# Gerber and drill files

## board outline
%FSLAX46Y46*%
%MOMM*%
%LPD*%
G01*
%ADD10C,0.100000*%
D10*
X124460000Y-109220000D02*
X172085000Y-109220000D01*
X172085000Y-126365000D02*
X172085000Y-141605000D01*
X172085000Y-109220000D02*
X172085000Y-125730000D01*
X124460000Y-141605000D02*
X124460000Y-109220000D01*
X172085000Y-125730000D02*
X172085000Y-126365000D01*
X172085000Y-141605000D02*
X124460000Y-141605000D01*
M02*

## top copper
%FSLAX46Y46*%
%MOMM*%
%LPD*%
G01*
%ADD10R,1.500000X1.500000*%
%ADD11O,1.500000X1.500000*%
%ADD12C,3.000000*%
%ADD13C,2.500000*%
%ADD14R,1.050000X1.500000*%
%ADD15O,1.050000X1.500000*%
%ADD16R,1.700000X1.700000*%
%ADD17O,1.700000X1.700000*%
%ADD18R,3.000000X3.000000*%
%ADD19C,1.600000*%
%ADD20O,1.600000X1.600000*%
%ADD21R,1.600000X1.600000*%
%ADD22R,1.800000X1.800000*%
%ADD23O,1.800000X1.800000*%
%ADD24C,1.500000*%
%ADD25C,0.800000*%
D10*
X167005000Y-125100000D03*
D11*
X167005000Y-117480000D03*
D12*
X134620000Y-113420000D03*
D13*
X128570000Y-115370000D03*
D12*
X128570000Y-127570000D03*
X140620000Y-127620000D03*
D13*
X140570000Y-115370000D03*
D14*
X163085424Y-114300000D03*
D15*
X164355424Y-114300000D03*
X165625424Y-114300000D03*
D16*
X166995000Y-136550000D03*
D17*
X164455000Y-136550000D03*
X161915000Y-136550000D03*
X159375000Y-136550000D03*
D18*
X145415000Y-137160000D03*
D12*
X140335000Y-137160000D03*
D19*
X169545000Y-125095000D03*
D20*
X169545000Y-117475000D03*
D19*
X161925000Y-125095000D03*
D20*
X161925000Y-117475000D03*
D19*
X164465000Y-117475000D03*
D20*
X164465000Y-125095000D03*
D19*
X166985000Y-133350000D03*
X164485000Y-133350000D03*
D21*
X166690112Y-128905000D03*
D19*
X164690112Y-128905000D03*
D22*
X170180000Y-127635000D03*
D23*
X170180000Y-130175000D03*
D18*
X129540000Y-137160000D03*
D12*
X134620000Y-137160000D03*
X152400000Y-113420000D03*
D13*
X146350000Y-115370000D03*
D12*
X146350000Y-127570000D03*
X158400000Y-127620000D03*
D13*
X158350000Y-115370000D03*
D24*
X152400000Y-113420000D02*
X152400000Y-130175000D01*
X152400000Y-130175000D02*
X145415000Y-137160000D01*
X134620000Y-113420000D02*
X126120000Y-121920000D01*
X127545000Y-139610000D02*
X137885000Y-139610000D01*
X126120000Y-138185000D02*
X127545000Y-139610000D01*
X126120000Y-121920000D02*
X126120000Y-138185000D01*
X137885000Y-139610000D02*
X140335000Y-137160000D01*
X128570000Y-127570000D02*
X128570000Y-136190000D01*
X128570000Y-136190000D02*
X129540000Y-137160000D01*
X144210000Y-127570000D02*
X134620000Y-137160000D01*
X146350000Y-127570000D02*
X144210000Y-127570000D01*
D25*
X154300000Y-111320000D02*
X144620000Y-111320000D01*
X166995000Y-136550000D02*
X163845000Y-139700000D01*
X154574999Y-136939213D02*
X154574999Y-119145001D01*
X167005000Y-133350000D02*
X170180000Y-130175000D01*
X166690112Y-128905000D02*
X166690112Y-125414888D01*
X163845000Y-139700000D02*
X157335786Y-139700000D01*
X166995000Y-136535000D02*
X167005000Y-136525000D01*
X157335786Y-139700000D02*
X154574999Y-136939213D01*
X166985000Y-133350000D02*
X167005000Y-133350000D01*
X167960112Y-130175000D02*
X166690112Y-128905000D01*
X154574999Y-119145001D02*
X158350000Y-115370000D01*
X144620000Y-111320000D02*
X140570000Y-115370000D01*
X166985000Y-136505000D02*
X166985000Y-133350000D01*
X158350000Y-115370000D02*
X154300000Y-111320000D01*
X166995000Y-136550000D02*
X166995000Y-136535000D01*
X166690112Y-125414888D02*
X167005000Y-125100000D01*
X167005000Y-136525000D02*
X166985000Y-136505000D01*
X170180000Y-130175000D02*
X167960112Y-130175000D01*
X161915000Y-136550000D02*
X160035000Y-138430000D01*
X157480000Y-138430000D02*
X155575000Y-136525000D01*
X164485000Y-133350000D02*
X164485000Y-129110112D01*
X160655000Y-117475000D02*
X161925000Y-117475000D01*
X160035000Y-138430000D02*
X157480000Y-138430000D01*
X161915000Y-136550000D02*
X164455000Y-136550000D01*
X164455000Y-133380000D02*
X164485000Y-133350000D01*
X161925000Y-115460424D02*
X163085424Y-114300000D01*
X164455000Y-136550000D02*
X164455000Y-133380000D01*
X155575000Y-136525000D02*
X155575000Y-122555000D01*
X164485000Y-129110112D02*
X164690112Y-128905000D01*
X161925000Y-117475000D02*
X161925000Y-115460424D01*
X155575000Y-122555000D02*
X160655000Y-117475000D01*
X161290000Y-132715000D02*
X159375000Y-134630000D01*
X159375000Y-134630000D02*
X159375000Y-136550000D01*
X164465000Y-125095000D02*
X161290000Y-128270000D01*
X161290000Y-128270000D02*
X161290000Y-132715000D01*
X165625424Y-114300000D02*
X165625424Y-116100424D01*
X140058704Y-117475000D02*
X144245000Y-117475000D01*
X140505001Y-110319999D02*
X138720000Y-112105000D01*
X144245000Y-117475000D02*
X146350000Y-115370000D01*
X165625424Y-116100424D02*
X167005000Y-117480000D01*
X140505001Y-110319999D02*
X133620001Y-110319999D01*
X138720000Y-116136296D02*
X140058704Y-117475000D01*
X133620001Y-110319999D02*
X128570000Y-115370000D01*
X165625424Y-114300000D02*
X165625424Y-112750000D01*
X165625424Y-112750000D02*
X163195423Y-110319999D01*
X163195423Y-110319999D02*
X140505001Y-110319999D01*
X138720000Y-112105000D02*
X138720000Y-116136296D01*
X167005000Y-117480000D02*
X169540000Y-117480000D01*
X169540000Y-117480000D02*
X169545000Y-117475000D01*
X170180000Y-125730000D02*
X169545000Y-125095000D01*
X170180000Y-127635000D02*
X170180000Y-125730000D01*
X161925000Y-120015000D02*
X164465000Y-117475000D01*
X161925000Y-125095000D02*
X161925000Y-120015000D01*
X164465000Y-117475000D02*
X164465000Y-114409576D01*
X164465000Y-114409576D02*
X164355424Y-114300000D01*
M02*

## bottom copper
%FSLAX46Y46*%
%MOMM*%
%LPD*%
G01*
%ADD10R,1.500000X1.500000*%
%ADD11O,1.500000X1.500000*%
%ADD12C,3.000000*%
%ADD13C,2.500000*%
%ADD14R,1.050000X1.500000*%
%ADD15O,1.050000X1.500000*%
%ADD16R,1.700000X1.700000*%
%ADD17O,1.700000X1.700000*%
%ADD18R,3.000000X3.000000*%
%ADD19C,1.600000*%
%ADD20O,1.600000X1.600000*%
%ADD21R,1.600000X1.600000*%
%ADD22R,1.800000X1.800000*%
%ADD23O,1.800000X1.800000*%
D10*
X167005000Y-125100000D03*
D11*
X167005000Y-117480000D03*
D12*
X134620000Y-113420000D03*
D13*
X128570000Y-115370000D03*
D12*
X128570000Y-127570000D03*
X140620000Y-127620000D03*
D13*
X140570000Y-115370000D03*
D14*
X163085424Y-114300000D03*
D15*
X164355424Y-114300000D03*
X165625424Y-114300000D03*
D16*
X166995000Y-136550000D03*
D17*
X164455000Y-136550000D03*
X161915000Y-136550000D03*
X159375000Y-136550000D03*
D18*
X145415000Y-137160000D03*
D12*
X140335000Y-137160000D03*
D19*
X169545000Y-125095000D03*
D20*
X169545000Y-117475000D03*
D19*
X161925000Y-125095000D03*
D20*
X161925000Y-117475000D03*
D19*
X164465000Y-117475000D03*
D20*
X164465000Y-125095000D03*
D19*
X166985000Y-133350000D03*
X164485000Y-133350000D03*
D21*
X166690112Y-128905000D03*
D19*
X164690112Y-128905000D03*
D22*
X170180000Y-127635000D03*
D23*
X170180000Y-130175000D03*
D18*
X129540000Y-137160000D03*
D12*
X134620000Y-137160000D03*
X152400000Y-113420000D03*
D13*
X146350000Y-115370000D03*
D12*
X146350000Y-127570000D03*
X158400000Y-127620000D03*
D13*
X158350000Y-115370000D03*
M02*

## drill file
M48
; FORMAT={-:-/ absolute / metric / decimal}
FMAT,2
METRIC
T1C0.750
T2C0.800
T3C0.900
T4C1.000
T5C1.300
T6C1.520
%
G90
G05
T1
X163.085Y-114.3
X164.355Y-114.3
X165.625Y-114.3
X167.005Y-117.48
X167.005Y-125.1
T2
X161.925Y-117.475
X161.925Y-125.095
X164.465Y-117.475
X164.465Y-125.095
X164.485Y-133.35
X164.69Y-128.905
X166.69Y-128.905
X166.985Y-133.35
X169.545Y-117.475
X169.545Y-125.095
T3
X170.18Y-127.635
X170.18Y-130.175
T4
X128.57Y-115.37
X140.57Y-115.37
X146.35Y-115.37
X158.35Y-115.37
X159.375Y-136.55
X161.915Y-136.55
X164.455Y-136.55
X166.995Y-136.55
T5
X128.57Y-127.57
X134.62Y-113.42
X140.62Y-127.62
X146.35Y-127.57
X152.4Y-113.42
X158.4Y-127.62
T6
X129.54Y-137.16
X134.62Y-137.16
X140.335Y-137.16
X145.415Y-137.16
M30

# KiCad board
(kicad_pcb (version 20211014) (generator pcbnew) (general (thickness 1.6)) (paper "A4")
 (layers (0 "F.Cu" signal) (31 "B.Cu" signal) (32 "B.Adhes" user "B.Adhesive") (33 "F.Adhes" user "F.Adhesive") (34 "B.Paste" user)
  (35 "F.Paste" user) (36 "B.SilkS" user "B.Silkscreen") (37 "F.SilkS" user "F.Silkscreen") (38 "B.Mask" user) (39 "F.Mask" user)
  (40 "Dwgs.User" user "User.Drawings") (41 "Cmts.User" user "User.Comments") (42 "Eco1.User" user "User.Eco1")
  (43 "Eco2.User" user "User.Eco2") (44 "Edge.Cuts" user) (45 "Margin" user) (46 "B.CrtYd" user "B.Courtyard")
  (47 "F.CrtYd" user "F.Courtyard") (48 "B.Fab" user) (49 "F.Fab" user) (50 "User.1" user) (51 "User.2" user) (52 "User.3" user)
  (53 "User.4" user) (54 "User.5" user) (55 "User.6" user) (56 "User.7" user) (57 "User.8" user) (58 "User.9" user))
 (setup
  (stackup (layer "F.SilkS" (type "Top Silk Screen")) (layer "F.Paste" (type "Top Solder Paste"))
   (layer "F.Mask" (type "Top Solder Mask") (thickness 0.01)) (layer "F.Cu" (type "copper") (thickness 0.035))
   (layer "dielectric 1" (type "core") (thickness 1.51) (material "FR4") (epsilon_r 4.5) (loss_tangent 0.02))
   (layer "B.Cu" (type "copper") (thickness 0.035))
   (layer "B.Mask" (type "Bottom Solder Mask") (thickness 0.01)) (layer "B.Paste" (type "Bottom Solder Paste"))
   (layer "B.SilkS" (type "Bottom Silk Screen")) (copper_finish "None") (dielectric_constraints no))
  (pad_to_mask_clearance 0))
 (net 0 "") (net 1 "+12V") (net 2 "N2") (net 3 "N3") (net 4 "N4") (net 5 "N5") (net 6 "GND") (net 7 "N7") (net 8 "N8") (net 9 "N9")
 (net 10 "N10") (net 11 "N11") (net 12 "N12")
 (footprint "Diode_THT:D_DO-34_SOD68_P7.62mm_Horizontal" (layer "F.Cu") (at 167.005 125.1 90)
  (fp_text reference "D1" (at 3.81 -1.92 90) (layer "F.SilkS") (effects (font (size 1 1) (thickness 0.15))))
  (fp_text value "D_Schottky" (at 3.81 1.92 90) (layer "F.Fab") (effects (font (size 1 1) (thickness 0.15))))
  (pad "1" thru_hole rect (at 0 0 90) (size 1.5 1.5) (drill 0.75) (layers *.Cu *.Mask) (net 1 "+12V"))
  (pad "2" thru_hole oval (at 7.62 0 90) (size 1.5 1.5) (drill 0.75) (layers *.Cu *.Mask) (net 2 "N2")))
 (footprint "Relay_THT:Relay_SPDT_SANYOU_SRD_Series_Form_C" (layer "F.Cu") (at 134.62 113.42 -90)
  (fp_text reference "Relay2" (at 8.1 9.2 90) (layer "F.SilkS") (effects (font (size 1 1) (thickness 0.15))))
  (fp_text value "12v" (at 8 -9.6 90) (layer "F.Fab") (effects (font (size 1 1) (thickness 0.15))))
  (pad "1" thru_hole circle (at 0 0) (size 3 3) (drill 1.3) (layers *.Cu *.Mask) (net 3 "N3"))
  (pad "2" thru_hole circle (at 1.95 6.05) (size 2.5 2.5) (drill 1) (layers *.Cu *.Mask) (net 2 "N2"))
  (pad "3" thru_hole circle (at 14.15 6.05) (size 3 3) (drill 1.3) (layers *.Cu *.Mask) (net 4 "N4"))
  (pad "4" thru_hole circle (at 14.2 -6) (size 3 3) (drill 1.3) (layers *.Cu *.Mask) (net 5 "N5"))
  (pad "5" thru_hole circle (at 1.95 -5.95) (size 2.5 2.5) (drill 1) (layers *.Cu *.Mask) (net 1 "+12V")))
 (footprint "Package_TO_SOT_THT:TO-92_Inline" (layer "F.Cu") (at 163.085424 114.3)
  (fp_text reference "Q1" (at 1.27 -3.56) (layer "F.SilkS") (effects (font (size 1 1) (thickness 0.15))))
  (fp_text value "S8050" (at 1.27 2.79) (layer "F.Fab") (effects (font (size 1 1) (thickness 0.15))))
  (pad "1" thru_hole rect (at 0 0) (size 1.05 1.5) (drill 0.75) (layers *.Cu *.Mask) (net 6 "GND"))
  (pad "2" thru_hole oval (at 1.27 0) (size 1.05 1.5) (drill 0.75) (layers *.Cu *.Mask) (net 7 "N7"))
  (pad "3" thru_hole oval (at 2.54 0) (size 1.05 1.5) (drill 0.75) (layers *.Cu *.Mask) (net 2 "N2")))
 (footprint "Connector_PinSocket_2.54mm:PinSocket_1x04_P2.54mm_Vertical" (layer "F.Cu") (at 166.995 136.55 -90)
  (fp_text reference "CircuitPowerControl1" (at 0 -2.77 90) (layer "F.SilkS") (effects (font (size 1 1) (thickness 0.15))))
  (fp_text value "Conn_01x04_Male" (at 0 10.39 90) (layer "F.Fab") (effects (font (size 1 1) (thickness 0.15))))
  (pad "1" thru_hole rect (at 0 0 270) (size 1.7 1.7) (drill 1) (layers *.Cu *.Mask) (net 1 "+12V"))
  (pad "2" thru_hole oval (at 0 2.54 270) (size 1.7 1.7) (drill 1) (layers *.Cu *.Mask) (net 6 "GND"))
  (pad "3" thru_hole oval (at 0 5.08 270) (size 1.7 1.7) (drill 1) (layers *.Cu *.Mask) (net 6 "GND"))
  (pad "4" thru_hole oval (at 0 7.62 270) (size 1.7 1.7) (drill 1) (layers *.Cu *.Mask) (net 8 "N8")))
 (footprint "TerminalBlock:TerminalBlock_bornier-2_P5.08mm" (layer "F.Cu") (at 145.415 137.16 180)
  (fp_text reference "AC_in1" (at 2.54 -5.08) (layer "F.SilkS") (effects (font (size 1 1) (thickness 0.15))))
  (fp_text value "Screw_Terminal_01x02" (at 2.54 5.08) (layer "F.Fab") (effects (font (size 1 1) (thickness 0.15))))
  (pad "1" thru_hole rect (at 0 0 180) (size 3 3) (drill 1.52) (layers *.Cu *.Mask) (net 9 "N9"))
  (pad "2" thru_hole circle (at 5.08 0 180) (size 3 3) (drill 1.52) (layers *.Cu *.Mask) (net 3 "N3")))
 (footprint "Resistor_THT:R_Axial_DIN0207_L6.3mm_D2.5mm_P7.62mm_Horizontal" (layer "F.Cu") (at 169.545 125.095 90)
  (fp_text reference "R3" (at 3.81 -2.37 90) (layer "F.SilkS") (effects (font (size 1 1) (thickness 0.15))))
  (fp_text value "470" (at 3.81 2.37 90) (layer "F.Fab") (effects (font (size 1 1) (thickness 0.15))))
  (pad "1" thru_hole circle (at 0 0 90) (size 1.6 1.6) (drill 0.8) (layers *.Cu *.Mask) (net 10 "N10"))
  (pad "2" thru_hole oval (at 7.62 0 90) (size 1.6 1.6) (drill 0.8) (layers *.Cu *.Mask) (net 2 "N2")))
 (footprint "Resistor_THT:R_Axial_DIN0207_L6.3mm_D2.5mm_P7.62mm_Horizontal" (layer "F.Cu") (at 161.925 125.095 90)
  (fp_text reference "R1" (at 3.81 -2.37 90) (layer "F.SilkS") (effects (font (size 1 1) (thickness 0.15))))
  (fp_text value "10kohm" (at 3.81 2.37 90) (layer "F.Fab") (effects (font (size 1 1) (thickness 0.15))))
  (pad "1" thru_hole circle (at 0 0 90) (size 1.6 1.6) (drill 0.8) (layers *.Cu *.Mask) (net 7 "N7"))
  (pad "2" thru_hole oval (at 7.62 0 90) (size 1.6 1.6) (drill 0.8) (layers *.Cu *.Mask) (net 6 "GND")))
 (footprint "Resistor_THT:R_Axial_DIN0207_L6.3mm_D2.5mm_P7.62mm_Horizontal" (layer "F.Cu") (at 164.465 117.475 -90)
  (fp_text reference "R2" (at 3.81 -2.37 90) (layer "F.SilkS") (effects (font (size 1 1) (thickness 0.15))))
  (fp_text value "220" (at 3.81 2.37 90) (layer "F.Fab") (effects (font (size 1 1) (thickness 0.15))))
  (pad "1" thru_hole circle (at 0 0 270) (size 1.6 1.6) (drill 0.8) (layers *.Cu *.Mask) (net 7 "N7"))
  (pad "2" thru_hole oval (at 7.62 0 270) (size 1.6 1.6) (drill 0.8) (layers *.Cu *.Mask) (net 8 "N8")))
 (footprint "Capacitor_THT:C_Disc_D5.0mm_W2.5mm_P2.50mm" (layer "F.Cu") (at 166.985 133.35 180)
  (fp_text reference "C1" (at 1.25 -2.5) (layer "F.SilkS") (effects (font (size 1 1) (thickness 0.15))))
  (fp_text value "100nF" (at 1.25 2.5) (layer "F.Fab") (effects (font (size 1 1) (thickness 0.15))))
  (pad "1" thru_hole circle (at 0 0 180) (size 1.6 1.6) (drill 0.8) (layers *.Cu *.Mask) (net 1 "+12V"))
  (pad "2" thru_hole circle (at 2.5 0 180) (size 1.6 1.6) (drill 0.8) (layers *.Cu *.Mask) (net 6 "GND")))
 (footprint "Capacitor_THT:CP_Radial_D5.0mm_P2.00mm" (layer "F.Cu") (at 166.690112 128.905 180)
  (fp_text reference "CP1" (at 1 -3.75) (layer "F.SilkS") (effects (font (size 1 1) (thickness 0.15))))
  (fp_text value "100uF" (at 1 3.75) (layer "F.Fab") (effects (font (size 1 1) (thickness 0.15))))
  (pad "1" thru_hole rect (at 0 0 180) (size 1.6 1.6) (drill 0.8) (layers *.Cu *.Mask) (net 1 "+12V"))
  (pad "2" thru_hole circle (at 2 0 180) (size 1.6 1.6) (drill 0.8) (layers *.Cu *.Mask) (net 6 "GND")))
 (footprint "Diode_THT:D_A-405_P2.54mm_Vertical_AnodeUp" (layer "F.Cu") (at 170.18 127.635 -90)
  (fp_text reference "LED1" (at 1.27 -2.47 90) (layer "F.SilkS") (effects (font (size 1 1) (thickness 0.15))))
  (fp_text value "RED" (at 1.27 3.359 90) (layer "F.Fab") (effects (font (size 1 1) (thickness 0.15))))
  (pad "1" thru_hole rect (at 0 0 270) (size 1.8 1.8) (drill 0.9) (layers *.Cu *.Mask) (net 10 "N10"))
  (pad "2" thru_hole oval (at 2.54 0 270) (size 1.8 1.8) (drill 0.9) (layers *.Cu *.Mask) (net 1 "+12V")))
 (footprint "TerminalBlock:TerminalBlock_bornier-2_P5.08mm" (layer "F.Cu") (at 129.54 137.16)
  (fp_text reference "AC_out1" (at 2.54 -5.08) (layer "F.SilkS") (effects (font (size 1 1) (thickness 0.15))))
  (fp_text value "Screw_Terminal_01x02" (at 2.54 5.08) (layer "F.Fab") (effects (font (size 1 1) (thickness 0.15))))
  (pad "1" thru_hole rect (at 0 0) (size 3 3) (drill 1.52) (layers *.Cu *.Mask) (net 4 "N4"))
  (pad "2" thru_hole circle (at 5.08 0) (size 3 3) (drill 1.52) (layers *.Cu *.Mask) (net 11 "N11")))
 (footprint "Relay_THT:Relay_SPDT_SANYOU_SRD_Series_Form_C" (layer "F.Cu") (at 152.4 113.42 -90)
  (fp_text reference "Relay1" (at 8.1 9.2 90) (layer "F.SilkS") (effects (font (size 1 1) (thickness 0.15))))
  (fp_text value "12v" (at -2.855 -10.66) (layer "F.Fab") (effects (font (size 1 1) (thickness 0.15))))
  (pad "1" thru_hole circle (at 0 0) (size 3 3) (drill 1.3) (layers *.Cu *.Mask) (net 9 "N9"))
  (pad "2" thru_hole circle (at 1.95 6.05) (size 2.5 2.5) (drill 1) (layers *.Cu *.Mask) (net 2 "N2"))
  (pad "3" thru_hole circle (at 14.15 6.05) (size 3 3) (drill 1.3) (layers *.Cu *.Mask) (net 11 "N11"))
  (pad "4" thru_hole circle (at 14.2 -6) (size 3 3) (drill 1.3) (layers *.Cu *.Mask) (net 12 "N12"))
  (pad "5" thru_hole circle (at 1.95 -5.95) (size 2.5 2.5) (drill 1) (layers *.Cu *.Mask) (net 1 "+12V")))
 (gr_line (start 124.46 109.22) (end 172.085 109.22) (layer "Edge.Cuts") (width 0.1))
 (gr_line (start 172.085 126.365) (end 172.085 141.605) (layer "Edge.Cuts") (width 0.1))
 (gr_line (start 172.085 109.22) (end 172.085 125.73) (layer "Edge.Cuts") (width 0.1))
 (gr_line (start 124.46 141.605) (end 124.46 109.22) (layer "Edge.Cuts") (width 0.1))
 (gr_line (start 172.085 125.73) (end 172.085 126.365) (layer "Edge.Cuts") (width 0.1))
 (gr_line (start 172.085 141.605) (end 124.46 141.605) (layer "Edge.Cuts") (width 0.1))
 (segment (start 152.4 113.42) (end 152.4 130.175) (width 1.5) (layer "F.Cu") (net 9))
 (segment (start 152.4 130.175) (end 145.415 137.16) (width 1.5) (layer "F.Cu") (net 9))
 (segment (start 134.62 113.42) (end 126.12 121.92) (width 1.5) (layer "F.Cu") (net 3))
 (segment (start 127.545 139.61) (end 137.885 139.61) (width 1.5) (layer "F.Cu") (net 3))
 (segment (start 126.12 138.185) (end 127.545 139.61) (width 1.5) (layer "F.Cu") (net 3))
 (segment (start 126.12 121.92) (end 126.12 138.185) (width 1.5) (layer "F.Cu") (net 3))
 (segment (start 137.885 139.61) (end 140.335 137.16) (width 1.5) (layer "F.Cu") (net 3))
 (segment (start 128.57 127.57) (end 128.57 136.19) (width 1.5) (layer "F.Cu") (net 4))
 (segment (start 128.57 136.19) (end 129.54 137.16) (width 1.5) (layer "F.Cu") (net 4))
 (segment (start 144.21 127.57) (end 134.62 137.16) (width 1.5) (layer "F.Cu") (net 11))
 (segment (start 146.35 127.57) (end 144.21 127.57) (width 1.5) (layer "F.Cu") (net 11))
 (segment (start 154.3 111.32) (end 144.62 111.32) (width 0.8) (layer "F.Cu") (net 1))
 (segment (start 166.995 136.55) (end 163.845 139.7) (width 0.8) (layer "F.Cu") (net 1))
 (segment (start 154.574999 136.939213) (end 154.574999 119.145001) (width 0.8) (layer "F.Cu") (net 1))
 (segment (start 167.005 133.35) (end 170.18 130.175) (width 0.8) (layer "F.Cu") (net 1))
 (segment (start 166.690112 128.905) (end 166.690112 125.414888) (width 0.8) (layer "F.Cu") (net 1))
 (segment (start 163.845 139.7) (end 157.335786 139.7) (width 0.8) (layer "F.Cu") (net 1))
 (segment (start 166.995 136.535) (end 167.005 136.525) (width 0.8) (layer "F.Cu") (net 1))
 (segment (start 157.335786 139.7) (end 154.574999 136.939213) (width 0.8) (layer "F.Cu") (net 1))
 (segment (start 166.985 133.35) (end 167.005 133.35) (width 0.8) (layer "F.Cu") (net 1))
 (segment (start 167.960112 130.175) (end 166.690112 128.905) (width 0.8) (layer "F.Cu") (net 1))
 (segment (start 154.574999 119.145001) (end 158.35 115.37) (width 0.8) (layer "F.Cu") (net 1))
 (segment (start 144.62 111.32) (end 140.57 115.37) (width 0.8) (layer "F.Cu") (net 1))
 (segment (start 166.985 136.505) (end 166.985 133.35) (width 0.8) (layer "F.Cu") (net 1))
 (segment (start 158.35 115.37) (end 154.3 111.32) (width 0.8) (layer "F.Cu") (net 1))
 (segment (start 166.995 136.55) (end 166.995 136.535) (width 0.8) (layer "F.Cu") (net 1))
 (segment (start 166.690112 125.414888) (end 167.005 125.1) (width 0.8) (layer "F.Cu") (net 1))
 (segment (start 167.005 136.525) (end 166.985 136.505) (width 0.8) (layer "F.Cu") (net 1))
 (segment (start 170.18 130.175) (end 167.960112 130.175) (width 0.8) (layer "F.Cu") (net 1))
 (segment (start 161.915 136.55) (end 160.035 138.43) (width 0.8) (layer "F.Cu") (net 6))
 (segment (start 157.48 138.43) (end 155.575 136.525) (width 0.8) (layer "F.Cu") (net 6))
 (segment (start 164.485 133.35) (end 164.485 129.110112) (width 0.8) (layer "F.Cu") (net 6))
 (segment (start 160.655 117.475) (end 161.925 117.475) (width 0.8) (layer "F.Cu") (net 6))
 (segment (start 160.035 138.43) (end 157.48 138.43) (width 0.8) (layer "F.Cu") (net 6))
 (segment (start 161.915 136.55) (end 164.455 136.55) (width 0.8) (layer "F.Cu") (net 6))
 (segment (start 164.455 133.38) (end 164.485 133.35) (width 0.8) (layer "F.Cu") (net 6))
 (segment (start 161.925 115.460424) (end 163.085424 114.3) (width 0.8) (layer "F.Cu") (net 6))
 (segment (start 164.455 136.55) (end 164.455 133.38) (width 0.8) (layer "F.Cu") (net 6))
 (segment (start 155.575 136.525) (end 155.575 122.555) (width 0.8) (layer "F.Cu") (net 6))
 (segment (start 164.485 129.110112) (end 164.690112 128.905) (width 0.8) (layer "F.Cu") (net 6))
 (segment (start 161.925 117.475) (end 161.925 115.460424) (width 0.8) (layer "F.Cu") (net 6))
 (segment (start 155.575 122.555) (end 160.655 117.475) (width 0.8) (layer "F.Cu") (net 6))
 (segment (start 161.29 132.715) (end 159.375 134.63) (width 0.8) (layer "F.Cu") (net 8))
 (segment (start 159.375 134.63) (end 159.375 136.55) (width 0.8) (layer "F.Cu") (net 8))
 (segment (start 164.465 125.095) (end 161.29 128.27) (width 0.8) (layer "F.Cu") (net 8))
 (segment (start 161.29 128.27) (end 161.29 132.715) (width 0.8) (layer "F.Cu") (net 8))
 (segment (start 165.625424 114.3) (end 165.625424 116.100424) (width 0.8) (layer "F.Cu") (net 2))
 (segment (start 140.058704 117.475) (end 144.245 117.475) (width 0.8) (layer "F.Cu") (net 2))
 (segment (start 140.505001 110.319999) (end 138.72 112.105) (width 0.8) (layer "F.Cu") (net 2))
 (segment (start 144.245 117.475) (end 146.35 115.37) (width 0.8) (layer "F.Cu") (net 2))
 (segment (start 165.625424 116.100424) (end 167.005 117.48) (width 0.8) (layer "F.Cu") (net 2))
 (segment (start 140.505001 110.319999) (end 133.620001 110.319999) (width 0.8) (layer "F.Cu") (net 2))
 (segment (start 138.72 116.136296) (end 140.058704 117.475) (width 0.8) (layer "F.Cu") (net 2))
 (segment (start 133.620001 110.319999) (end 128.57 115.37) (width 0.8) (layer "F.Cu") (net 2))
 (segment (start 165.625424 114.3) (end 165.625424 112.75) (width 0.8) (layer "F.Cu") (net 2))
 (segment (start 165.625424 112.75) (end 163.195423 110.319999) (width 0.8) (layer "F.Cu") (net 2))
 (segment (start 163.195423 110.319999) (end 140.505001 110.319999) (width 0.8) (layer "F.Cu") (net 2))
 (segment (start 138.72 112.105) (end 138.72 116.136296) (width 0.8) (layer "F.Cu") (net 2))
 (segment (start 167.005 117.48) (end 169.54 117.48) (width 0.8) (layer "F.Cu") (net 2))
 (segment (start 169.54 117.48) (end 169.545 117.475) (width 0.8) (layer "F.Cu") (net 2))
 (segment (start 170.18 125.73) (end 169.545 125.095) (width 0.8) (layer "F.Cu") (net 10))
 (segment (start 170.18 127.635) (end 170.18 125.73) (width 0.8) (layer "F.Cu") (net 10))
 (segment (start 161.925 120.015) (end 164.465 117.475) (width 0.8) (layer "F.Cu") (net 7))
 (segment (start 161.925 125.095) (end 161.925 120.015) (width 0.8) (layer "F.Cu") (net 7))
 (segment (start 164.465 117.475) (end 164.465 114.409576) (width 0.8) (layer "F.Cu") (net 7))
 (segment (start 164.465 114.409576) (end 164.355424 114.3) (width 0.8) (layer "F.Cu") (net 7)))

